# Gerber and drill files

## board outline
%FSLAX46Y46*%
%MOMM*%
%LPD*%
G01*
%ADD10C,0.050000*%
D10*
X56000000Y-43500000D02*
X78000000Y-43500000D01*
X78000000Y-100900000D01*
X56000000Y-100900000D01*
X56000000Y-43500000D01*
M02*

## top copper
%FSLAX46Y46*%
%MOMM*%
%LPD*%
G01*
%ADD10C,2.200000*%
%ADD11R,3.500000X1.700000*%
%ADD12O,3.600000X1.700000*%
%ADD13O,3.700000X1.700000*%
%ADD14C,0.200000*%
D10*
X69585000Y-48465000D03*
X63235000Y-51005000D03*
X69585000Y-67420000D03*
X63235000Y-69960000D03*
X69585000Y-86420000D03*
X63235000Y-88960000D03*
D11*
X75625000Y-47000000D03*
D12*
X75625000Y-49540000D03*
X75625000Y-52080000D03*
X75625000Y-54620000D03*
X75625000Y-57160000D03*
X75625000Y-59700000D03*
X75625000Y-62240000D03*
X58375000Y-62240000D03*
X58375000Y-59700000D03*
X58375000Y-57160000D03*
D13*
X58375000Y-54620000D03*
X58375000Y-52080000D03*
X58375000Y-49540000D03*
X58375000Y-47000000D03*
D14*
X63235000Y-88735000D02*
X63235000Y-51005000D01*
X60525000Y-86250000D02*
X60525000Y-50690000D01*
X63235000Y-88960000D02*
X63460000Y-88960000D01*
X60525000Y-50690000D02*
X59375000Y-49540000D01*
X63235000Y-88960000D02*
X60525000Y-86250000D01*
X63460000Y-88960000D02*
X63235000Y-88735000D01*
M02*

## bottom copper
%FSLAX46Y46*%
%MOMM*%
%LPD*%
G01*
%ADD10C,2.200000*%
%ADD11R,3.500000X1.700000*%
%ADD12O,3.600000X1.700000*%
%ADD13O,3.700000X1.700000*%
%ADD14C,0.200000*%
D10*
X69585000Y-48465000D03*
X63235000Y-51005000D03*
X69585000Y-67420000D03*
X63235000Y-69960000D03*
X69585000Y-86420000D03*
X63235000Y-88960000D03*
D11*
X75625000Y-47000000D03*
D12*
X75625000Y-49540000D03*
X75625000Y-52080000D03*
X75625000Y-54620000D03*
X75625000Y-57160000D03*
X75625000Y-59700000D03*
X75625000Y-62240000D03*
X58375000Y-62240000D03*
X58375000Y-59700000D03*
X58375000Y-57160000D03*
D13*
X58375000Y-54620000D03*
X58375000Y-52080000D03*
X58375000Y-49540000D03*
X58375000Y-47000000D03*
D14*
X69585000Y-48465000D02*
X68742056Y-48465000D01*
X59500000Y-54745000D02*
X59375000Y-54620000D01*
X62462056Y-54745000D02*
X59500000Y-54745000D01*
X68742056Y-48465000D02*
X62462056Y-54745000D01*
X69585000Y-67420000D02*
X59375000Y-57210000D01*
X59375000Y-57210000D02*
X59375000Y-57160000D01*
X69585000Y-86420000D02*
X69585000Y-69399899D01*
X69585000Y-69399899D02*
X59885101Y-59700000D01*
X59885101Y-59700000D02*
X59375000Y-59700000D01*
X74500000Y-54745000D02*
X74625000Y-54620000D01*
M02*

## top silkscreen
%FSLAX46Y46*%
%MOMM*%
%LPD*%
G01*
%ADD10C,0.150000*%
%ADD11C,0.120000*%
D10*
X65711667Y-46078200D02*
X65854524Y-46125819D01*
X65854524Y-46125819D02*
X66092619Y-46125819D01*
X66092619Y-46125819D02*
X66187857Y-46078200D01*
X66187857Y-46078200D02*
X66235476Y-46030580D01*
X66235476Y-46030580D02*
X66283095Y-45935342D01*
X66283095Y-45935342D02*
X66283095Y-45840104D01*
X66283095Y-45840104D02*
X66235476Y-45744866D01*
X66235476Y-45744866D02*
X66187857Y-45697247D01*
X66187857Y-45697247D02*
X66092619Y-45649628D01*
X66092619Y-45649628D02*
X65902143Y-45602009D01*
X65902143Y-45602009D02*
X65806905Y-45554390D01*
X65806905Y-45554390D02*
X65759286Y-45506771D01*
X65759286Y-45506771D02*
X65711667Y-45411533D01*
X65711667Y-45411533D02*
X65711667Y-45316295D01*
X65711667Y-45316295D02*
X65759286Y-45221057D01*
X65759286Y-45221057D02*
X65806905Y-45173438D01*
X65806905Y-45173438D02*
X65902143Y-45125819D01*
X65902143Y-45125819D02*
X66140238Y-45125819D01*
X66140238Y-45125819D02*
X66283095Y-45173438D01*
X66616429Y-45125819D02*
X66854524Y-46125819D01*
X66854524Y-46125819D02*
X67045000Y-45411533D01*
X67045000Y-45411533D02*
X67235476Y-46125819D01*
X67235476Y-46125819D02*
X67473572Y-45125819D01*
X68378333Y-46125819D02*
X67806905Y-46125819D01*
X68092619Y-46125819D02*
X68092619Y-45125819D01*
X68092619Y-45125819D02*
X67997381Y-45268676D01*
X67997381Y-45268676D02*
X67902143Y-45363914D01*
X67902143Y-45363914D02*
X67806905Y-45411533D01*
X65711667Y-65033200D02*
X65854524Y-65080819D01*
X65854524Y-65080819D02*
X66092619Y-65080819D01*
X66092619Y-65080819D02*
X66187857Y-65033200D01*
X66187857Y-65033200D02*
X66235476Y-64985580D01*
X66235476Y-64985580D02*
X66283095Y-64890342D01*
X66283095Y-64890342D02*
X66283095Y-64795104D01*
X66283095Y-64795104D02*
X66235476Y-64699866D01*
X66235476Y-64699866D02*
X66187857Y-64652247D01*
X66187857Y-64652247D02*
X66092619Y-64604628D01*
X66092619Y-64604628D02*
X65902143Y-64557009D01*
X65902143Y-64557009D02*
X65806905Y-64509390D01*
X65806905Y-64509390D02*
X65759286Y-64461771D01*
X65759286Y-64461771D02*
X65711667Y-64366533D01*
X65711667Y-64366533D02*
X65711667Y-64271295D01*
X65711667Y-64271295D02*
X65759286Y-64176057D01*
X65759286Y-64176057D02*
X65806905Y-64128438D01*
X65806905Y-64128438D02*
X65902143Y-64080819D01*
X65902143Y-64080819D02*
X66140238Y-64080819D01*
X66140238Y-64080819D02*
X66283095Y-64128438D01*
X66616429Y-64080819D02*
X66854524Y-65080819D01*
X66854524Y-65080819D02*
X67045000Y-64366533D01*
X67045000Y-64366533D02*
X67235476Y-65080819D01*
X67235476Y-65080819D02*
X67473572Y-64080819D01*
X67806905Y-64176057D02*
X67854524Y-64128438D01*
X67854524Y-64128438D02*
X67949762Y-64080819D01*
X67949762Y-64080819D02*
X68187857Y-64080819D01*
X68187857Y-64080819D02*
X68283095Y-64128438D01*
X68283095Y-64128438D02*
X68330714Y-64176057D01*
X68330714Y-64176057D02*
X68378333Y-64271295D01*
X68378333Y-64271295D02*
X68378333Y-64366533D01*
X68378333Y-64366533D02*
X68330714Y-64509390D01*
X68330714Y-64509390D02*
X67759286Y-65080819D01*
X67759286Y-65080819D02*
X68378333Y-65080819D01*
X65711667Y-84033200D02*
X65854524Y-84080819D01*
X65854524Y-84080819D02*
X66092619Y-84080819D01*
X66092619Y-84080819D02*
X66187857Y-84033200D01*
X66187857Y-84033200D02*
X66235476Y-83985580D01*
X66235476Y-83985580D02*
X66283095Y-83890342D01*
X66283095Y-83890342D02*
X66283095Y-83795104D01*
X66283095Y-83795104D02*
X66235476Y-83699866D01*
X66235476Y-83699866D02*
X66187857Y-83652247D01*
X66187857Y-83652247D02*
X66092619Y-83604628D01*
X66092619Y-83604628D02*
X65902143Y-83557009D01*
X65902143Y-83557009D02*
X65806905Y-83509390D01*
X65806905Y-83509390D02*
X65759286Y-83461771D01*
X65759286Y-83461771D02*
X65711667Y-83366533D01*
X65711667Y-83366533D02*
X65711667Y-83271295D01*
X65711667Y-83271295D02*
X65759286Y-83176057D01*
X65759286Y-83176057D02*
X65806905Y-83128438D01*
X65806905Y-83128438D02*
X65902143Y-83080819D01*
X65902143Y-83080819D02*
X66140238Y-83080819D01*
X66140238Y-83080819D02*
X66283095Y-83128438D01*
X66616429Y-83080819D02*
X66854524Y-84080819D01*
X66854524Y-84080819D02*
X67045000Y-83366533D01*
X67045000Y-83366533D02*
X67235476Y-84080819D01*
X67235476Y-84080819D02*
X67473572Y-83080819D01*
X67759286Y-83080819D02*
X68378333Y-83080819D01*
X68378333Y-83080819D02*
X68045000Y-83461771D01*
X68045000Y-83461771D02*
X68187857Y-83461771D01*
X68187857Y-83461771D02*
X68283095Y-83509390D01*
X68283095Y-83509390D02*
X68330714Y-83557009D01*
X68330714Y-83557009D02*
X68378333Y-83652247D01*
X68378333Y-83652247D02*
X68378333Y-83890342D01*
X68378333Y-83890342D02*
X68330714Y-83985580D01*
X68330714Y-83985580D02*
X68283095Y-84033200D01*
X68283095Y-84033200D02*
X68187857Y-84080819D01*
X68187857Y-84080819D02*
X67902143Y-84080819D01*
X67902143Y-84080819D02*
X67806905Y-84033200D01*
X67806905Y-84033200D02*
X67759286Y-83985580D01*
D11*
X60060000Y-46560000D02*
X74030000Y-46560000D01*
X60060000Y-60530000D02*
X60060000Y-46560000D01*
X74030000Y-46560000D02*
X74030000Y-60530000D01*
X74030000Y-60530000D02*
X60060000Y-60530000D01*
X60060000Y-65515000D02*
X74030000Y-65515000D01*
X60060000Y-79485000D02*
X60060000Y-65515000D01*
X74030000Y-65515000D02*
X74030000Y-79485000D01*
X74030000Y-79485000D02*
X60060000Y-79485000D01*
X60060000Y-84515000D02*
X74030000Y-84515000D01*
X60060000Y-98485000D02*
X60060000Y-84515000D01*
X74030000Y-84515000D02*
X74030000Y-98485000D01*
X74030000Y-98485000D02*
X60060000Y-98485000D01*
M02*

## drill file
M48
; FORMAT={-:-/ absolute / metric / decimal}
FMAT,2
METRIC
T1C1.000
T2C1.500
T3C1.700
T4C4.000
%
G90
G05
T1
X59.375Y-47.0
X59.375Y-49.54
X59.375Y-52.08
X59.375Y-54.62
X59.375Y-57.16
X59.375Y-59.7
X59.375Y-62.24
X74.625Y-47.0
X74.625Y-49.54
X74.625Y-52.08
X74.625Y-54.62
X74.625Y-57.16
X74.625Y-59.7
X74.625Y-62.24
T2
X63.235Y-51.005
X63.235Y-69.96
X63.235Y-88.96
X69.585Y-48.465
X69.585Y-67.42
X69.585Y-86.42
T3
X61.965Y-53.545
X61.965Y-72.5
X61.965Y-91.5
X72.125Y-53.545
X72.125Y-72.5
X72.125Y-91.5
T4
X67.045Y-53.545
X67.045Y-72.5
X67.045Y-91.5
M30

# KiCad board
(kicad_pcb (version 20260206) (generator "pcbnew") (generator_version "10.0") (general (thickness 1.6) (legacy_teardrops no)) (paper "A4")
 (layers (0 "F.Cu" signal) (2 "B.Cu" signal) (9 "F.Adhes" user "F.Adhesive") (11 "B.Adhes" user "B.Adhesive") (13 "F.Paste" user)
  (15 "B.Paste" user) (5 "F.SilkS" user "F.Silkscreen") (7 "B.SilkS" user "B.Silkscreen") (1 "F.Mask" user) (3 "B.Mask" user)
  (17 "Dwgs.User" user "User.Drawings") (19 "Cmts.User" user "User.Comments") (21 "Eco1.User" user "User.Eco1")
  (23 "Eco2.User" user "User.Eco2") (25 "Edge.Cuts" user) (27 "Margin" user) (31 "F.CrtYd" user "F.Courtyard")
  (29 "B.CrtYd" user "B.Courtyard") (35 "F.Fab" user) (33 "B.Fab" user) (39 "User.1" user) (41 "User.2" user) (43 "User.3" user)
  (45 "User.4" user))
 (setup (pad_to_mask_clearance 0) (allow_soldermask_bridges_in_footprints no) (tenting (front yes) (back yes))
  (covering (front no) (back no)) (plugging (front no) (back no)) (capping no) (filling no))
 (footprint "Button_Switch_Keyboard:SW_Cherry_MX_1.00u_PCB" (layer "F.Cu") (at 69.585 48.465)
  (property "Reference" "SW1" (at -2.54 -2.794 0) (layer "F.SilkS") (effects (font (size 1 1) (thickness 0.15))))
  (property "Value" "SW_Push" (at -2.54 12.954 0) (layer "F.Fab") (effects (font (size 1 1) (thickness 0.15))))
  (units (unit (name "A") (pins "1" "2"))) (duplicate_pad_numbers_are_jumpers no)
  (fp_line (start -9.525 -1.905) (end 4.445 -1.905) (stroke (width 0.12) (type solid)) (layer "F.SilkS"))
  (fp_line (start -9.525 12.065) (end -9.525 -1.905) (stroke (width 0.12) (type solid)) (layer "F.SilkS"))
  (fp_line (start 4.445 -1.905) (end 4.445 12.065) (stroke (width 0.12) (type solid)) (layer "F.SilkS"))
  (fp_line (start 4.445 12.065) (end -9.525 12.065) (stroke (width 0.12) (type solid)) (layer "F.SilkS"))
  (pad "" np_thru_hole circle (at -7.62 5.08) (size 1.7 1.7) (drill 1.7) (layers "*.Cu" "*.Mask"))
  (pad "" np_thru_hole circle (at -2.54 5.08) (size 4 4) (drill 4) (layers "*.Cu" "*.Mask"))
  (pad "" np_thru_hole circle (at 2.54 5.08) (size 1.7 1.7) (drill 1.7) (layers "*.Cu" "*.Mask"))
  (pad "1" thru_hole circle (at 0 0) (size 2.2 2.2) (drill 1.5) (layers "*.Cu" "*.Mask") (remove_unused_layers no)
   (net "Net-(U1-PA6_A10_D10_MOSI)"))
  (pad "2" thru_hole circle (at -6.35 2.54) (size 2.2 2.2) (drill 1.5) (layers "*.Cu" "*.Mask") (remove_unused_layers no) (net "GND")))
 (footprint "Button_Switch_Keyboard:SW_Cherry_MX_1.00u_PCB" (layer "F.Cu") (at 69.585 67.42)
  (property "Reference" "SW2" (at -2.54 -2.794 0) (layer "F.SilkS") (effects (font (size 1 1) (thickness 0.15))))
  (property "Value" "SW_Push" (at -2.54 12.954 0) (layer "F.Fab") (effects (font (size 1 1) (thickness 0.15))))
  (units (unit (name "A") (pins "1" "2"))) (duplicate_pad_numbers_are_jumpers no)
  (fp_line (start -9.525 -1.905) (end 4.445 -1.905) (stroke (width 0.12) (type solid)) (layer "F.SilkS"))
  (fp_line (start -9.525 12.065) (end -9.525 -1.905) (stroke (width 0.12) (type solid)) (layer "F.SilkS"))
  (fp_line (start 4.445 -1.905) (end 4.445 12.065) (stroke (width 0.12) (type solid)) (layer "F.SilkS"))
  (fp_line (start 4.445 12.065) (end -9.525 12.065) (stroke (width 0.12) (type solid)) (layer "F.SilkS"))
  (pad "" np_thru_hole circle (at -7.62 5.08) (size 1.7 1.7) (drill 1.7) (layers "*.Cu" "*.Mask"))
  (pad "" np_thru_hole circle (at -2.54 5.08) (size 4 4) (drill 4) (layers "*.Cu" "*.Mask"))
  (pad "" np_thru_hole circle (at 2.54 5.08) (size 1.7 1.7) (drill 1.7) (layers "*.Cu" "*.Mask"))
  (pad "1" thru_hole circle (at 0 0) (size 2.2 2.2) (drill 1.5) (layers "*.Cu" "*.Mask") (remove_unused_layers no)
   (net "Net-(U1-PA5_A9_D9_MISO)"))
  (pad "2" thru_hole circle (at -6.35 2.54) (size 2.2 2.2) (drill 1.5) (layers "*.Cu" "*.Mask") (remove_unused_layers no) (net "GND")))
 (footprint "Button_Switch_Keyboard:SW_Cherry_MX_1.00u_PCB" (layer "F.Cu") (at 69.585 86.42)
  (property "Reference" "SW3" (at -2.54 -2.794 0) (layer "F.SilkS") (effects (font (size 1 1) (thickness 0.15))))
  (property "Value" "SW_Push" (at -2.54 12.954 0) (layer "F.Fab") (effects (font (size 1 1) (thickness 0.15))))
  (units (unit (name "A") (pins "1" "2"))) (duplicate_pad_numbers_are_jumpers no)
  (fp_line (start -9.525 -1.905) (end 4.445 -1.905) (stroke (width 0.12) (type solid)) (layer "F.SilkS"))
  (fp_line (start -9.525 12.065) (end -9.525 -1.905) (stroke (width 0.12) (type solid)) (layer "F.SilkS"))
  (fp_line (start 4.445 -1.905) (end 4.445 12.065) (stroke (width 0.12) (type solid)) (layer "F.SilkS"))
  (fp_line (start 4.445 12.065) (end -9.525 12.065) (stroke (width 0.12) (type solid)) (layer "F.SilkS"))
  (pad "" np_thru_hole circle (at -7.62 5.08) (size 1.7 1.7) (drill 1.7) (layers "*.Cu" "*.Mask"))
  (pad "" np_thru_hole circle (at -2.54 5.08) (size 4 4) (drill 4) (layers "*.Cu" "*.Mask"))
  (pad "" np_thru_hole circle (at 2.54 5.08) (size 1.7 1.7) (drill 1.7) (layers "*.Cu" "*.Mask"))
  (pad "1" thru_hole circle (at 0 0) (size 2.2 2.2) (drill 1.5) (layers "*.Cu" "*.Mask") (remove_unused_layers no)
   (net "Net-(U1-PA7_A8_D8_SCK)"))
  (pad "2" thru_hole circle (at -6.35 2.54) (size 2.2 2.2) (drill 1.5) (layers "*.Cu" "*.Mask") (remove_unused_layers no) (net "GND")))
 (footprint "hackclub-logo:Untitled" (layer "B.Cu") (at 77 101 180)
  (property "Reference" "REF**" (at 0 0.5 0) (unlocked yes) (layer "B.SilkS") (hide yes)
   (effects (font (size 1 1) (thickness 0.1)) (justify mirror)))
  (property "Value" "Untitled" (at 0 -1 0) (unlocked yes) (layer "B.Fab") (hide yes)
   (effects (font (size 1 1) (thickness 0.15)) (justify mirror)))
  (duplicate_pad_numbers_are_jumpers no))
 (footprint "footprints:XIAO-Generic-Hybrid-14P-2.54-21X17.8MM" (layer "B.Cu") (at 67 54.62 180)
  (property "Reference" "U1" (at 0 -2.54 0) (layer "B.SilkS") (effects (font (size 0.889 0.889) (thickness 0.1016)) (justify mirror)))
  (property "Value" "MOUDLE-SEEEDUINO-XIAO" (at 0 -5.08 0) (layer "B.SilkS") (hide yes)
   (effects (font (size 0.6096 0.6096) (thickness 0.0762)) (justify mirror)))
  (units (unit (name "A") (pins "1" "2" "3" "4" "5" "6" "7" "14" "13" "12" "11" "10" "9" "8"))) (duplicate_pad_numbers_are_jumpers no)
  (pad "1" thru_hole rect (at -7.625 7.62 180) (size 3.5 1.7) (drill 1 (offset -1 0)) (layers "*.Cu" "*.Mask") (remove_unused_layers no)
   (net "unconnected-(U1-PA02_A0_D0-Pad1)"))
  (pad "2" thru_hole oval (at -7.625 5.08 180) (size 3.6 1.7) (drill 1 (offset -1 0)) (layers "*.Cu" "*.Mask") (remove_unused_layers no)
   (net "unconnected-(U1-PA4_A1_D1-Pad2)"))
  (pad "3" thru_hole oval (at -7.625 2.54 180) (size 3.6 1.7) (drill 1 (offset -1 0)) (layers "*.Cu" "*.Mask") (remove_unused_layers no)
   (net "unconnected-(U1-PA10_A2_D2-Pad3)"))
  (pad "4" thru_hole oval (at -7.625 0 180) (size 3.6 1.7) (drill 1 (offset -1 0)) (layers "*.Cu" "*.Mask") (remove_unused_layers no)
   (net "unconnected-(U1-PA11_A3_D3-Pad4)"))
  (pad "5" thru_hole oval (at -7.625 -2.54 180) (size 3.6 1.7) (drill 1 (offset -1 0)) (layers "*.Cu" "*.Mask") (remove_unused_layers no)
   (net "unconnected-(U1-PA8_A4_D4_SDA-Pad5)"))
  (pad "6" thru_hole oval (at -7.625 -5.08) (size 3.6 1.7) (drill 1 (offset 1 0)) (layers "*.Cu" "*.Mask") (remove_unused_layers no)
   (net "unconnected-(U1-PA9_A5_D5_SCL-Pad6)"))
  (pad "7" thru_hole oval (at -7.625 -7.62 180) (size 3.6 1.7) (drill 1 (offset -1 0)) (layers "*.Cu" "*.Mask") (remove_unused_layers no)
   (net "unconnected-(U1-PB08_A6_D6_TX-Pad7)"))
  (pad "8" thru_hole oval (at 7.625 -7.62 180) (size 3.6 1.7) (drill 1 (offset 1 0)) (layers "*.Cu" "*.Mask") (remove_unused_layers no)
   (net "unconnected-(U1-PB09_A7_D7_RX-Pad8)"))
  (pad "9" thru_hole oval (at 7.625 -5.08 180) (size 3.6 1.7) (drill 1 (offset 1 0)) (layers "*.Cu" "*.Mask") (remove_unused_layers no)
   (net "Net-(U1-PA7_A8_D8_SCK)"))
  (pad "10" thru_hole oval (at 7.625 -2.54 180) (size 3.6 1.7) (drill 1 (offset 1 0)) (layers "*.Cu" "*.Mask") (remove_unused_layers no)
   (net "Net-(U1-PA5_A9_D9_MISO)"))
  (pad "11" thru_hole oval (at 7.625 0 180) (size 3.7 1.7) (drill 1 (offset 1 0)) (layers "*.Cu" "*.Mask") (remove_unused_layers no)
   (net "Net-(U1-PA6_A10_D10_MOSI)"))
  (pad "12" thru_hole oval (at 7.625 2.54 180) (size 3.7 1.7) (drill 1 (offset 1 0)) (layers "*.Cu" "*.Mask") (remove_unused_layers no)
   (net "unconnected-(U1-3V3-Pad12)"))
  (pad "13" thru_hole oval (at 7.625 5.08 180) (size 3.7 1.7) (drill 1 (offset 1 0)) (layers "*.Cu" "*.Mask") (remove_unused_layers no)
   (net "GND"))
  (pad "14" thru_hole oval (at 7.625 7.62 180) (size 3.7 1.7) (drill 1 (offset 1 0)) (layers "*.Cu" "*.Mask") (remove_unused_layers no)
   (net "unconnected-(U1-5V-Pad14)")))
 (gr_rect (start 56 43.5) (end 78 100.9) (stroke (width 0.05) (type default)) (fill no) (layer "Edge.Cuts"))
 (segment (start 69.585 48.465) (end 68.742056 48.465) (width 0.2) (layer "B.Cu") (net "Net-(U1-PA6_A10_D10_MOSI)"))
 (segment (start 59.5 54.745) (end 59.375 54.62) (width 0.2) (layer "B.Cu") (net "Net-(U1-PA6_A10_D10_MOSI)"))
 (segment (start 62.462056 54.745) (end 59.5 54.745) (width 0.2) (layer "B.Cu") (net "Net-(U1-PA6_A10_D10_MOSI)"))
 (segment (start 68.742056 48.465) (end 62.462056 54.745) (width 0.2) (layer "B.Cu") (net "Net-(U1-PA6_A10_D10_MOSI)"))
 (segment (start 63.235 88.735) (end 63.235 51.005) (width 0.2) (layer "F.Cu") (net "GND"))
 (segment (start 60.525 86.25) (end 60.525 50.69) (width 0.2) (layer "F.Cu") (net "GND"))
 (segment (start 63.235 88.96) (end 63.46 88.96) (width 0.2) (layer "F.Cu") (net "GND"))
 (segment (start 60.525 50.69) (end 59.375 49.54) (width 0.2) (layer "F.Cu") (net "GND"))
 (segment (start 63.235 88.96) (end 60.525 86.25) (width 0.2) (layer "F.Cu") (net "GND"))
 (segment (start 63.46 88.96) (end 63.235 88.735) (width 0.2) (layer "F.Cu") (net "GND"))
 (segment (start 69.585 67.42) (end 59.375 57.21) (width 0.2) (layer "B.Cu") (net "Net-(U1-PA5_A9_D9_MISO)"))
 (segment (start 59.375 57.21) (end 59.375 57.16) (width 0.2) (layer "B.Cu") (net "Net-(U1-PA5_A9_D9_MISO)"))
 (segment (start 69.585 86.42) (end 69.585 69.399899) (width 0.2) (layer "B.Cu") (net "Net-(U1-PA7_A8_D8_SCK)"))
 (segment (start 69.585 69.399899) (end 59.885101 59.7) (width 0.2) (layer "B.Cu") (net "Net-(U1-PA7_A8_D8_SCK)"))
 (segment (start 59.885101 59.7) (end 59.375 59.7) (width 0.2) (layer "B.Cu") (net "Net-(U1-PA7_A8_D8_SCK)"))
 (segment (start 74.5 54.745) (end 74.625 54.62) (width 0.2) (layer "B.Cu") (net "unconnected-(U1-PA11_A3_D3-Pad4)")))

